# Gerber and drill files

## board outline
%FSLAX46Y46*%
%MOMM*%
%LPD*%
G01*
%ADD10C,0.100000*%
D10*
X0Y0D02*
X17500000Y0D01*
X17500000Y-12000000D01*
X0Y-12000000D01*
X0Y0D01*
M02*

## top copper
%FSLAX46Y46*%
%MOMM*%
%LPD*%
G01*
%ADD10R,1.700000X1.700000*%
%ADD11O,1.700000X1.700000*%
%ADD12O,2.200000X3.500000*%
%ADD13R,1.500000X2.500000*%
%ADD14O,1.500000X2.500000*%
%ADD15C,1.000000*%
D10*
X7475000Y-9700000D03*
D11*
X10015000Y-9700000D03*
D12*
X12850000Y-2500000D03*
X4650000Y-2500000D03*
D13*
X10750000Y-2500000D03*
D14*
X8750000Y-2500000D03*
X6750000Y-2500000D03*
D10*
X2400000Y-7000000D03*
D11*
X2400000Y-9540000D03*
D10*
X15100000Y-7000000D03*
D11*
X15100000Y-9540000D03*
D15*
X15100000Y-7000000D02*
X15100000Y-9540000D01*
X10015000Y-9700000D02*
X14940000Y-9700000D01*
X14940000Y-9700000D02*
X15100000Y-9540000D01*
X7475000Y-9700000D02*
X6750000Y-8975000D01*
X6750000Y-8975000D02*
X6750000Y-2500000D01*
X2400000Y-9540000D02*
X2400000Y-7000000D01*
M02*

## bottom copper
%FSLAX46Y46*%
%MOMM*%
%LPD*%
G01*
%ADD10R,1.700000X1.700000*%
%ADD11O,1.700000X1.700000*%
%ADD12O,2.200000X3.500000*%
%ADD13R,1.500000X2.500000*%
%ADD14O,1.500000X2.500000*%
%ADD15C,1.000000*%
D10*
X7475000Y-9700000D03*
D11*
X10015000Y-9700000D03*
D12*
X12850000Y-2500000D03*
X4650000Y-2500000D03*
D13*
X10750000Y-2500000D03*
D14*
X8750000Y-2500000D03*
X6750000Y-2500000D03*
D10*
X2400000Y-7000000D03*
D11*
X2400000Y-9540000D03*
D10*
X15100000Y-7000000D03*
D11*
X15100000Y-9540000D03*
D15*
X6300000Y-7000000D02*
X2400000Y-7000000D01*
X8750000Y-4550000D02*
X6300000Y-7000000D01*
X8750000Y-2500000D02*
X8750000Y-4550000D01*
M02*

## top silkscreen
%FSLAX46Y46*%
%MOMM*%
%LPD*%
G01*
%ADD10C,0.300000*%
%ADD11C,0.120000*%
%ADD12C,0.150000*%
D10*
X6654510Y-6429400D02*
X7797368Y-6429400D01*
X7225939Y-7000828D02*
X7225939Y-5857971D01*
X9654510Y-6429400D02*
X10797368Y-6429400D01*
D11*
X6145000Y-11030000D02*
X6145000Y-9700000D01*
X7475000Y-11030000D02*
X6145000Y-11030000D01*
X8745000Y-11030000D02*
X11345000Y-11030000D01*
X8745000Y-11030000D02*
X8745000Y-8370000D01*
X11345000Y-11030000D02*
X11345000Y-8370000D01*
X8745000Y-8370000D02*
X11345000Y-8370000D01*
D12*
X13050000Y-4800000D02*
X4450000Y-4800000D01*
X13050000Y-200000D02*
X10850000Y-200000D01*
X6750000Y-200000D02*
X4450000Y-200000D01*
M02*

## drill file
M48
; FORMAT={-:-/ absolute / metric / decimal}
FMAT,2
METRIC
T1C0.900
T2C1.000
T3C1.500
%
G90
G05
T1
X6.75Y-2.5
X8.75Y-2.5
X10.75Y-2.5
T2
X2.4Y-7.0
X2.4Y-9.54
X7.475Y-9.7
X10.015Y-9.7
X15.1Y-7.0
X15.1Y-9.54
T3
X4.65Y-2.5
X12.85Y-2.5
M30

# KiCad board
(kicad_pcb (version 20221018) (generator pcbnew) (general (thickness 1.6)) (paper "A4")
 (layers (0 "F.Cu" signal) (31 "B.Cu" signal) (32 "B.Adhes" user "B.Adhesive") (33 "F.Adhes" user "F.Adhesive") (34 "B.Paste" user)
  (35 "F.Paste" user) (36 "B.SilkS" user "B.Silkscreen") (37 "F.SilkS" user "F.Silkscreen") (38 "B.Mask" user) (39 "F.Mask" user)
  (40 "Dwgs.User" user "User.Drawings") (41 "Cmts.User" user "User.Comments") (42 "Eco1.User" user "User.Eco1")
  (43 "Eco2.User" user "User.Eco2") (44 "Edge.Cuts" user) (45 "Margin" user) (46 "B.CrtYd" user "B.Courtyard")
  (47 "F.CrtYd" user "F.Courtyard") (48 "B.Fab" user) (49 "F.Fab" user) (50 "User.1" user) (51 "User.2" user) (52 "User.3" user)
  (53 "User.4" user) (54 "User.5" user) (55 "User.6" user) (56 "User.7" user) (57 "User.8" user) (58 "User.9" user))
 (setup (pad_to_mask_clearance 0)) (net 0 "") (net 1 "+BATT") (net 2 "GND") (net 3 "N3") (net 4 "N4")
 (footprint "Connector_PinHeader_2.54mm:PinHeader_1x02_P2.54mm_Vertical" (layer "F.Cu") (at 7.475 9.7 90)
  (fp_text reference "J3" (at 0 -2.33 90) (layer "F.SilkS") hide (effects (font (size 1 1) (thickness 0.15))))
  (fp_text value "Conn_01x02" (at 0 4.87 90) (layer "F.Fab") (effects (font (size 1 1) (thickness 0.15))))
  (fp_line (start -1.33 -1.33) (end 0 -1.33) (stroke (width 0.12) (type solid)) (layer "F.SilkS"))
  (fp_line (start -1.33 0) (end -1.33 -1.33) (stroke (width 0.12) (type solid)) (layer "F.SilkS"))
  (fp_line (start -1.33 1.27) (end -1.33 3.87) (stroke (width 0.12) (type solid)) (layer "F.SilkS"))
  (fp_line (start -1.33 1.27) (end 1.33 1.27) (stroke (width 0.12) (type solid)) (layer "F.SilkS"))
  (fp_line (start -1.33 3.87) (end 1.33 3.87) (stroke (width 0.12) (type solid)) (layer "F.SilkS"))
  (fp_line (start 1.33 1.27) (end 1.33 3.87) (stroke (width 0.12) (type solid)) (layer "F.SilkS"))
  (pad "1" thru_hole rect (at 0 0 90) (size 1.7 1.7) (drill 1) (layers "*.Cu" "*.Mask") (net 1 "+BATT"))
  (pad "2" thru_hole oval (at 0 2.54 90) (size 1.7 1.7) (drill 1) (layers "*.Cu" "*.Mask") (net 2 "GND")))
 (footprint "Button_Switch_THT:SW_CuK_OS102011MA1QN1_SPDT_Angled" (layer "F.Cu") (at 10.75 2.5 180)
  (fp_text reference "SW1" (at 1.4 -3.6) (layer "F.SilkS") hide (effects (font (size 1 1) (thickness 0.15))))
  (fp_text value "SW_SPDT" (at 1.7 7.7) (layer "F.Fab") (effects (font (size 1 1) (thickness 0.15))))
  (fp_line (start -2.3 -2.3) (end 6.3 -2.3) (stroke (width 0.15) (type solid)) (layer "F.SilkS"))
  (fp_line (start -2.3 2.3) (end -0.1 2.3) (stroke (width 0.15) (type solid)) (layer "F.SilkS"))
  (fp_line (start 4 2.3) (end 6.3 2.3) (stroke (width 0.15) (type solid)) (layer "F.SilkS"))
  (pad "" thru_hole oval (at -2.1 0 180) (size 2.2 3.5) (drill 1.5) (layers "*.Cu" "*.Mask"))
  (pad "" thru_hole oval (at 6.1 0 180) (size 2.2 3.5) (drill 1.5) (layers "*.Cu" "*.Mask"))
  (pad "1" thru_hole rect (at 0 0 180) (size 1.5 2.5) (drill 0.9) (layers "*.Cu" "*.Mask") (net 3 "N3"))
  (pad "2" thru_hole oval (at 2 0 180) (size 1.5 2.5) (drill 0.9) (layers "*.Cu" "*.Mask") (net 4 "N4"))
  (pad "3" thru_hole oval (at 4 0 180) (size 1.5 2.5) (drill 0.9) (layers "*.Cu" "*.Mask") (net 1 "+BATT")))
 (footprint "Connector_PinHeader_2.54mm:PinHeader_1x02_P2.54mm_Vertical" (layer "B.Cu") (at 2.4 7 180)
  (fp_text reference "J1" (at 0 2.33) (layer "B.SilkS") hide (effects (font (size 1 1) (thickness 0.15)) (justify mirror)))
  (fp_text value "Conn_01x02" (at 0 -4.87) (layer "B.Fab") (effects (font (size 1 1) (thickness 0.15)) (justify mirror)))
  (pad "1" thru_hole rect (at 0 0 180) (size 1.7 1.7) (drill 1) (layers "*.Cu" "*.Mask") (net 4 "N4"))
  (pad "2" thru_hole oval (at 0 -2.54 180) (size 1.7 1.7) (drill 1) (layers "*.Cu" "*.Mask") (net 4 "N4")))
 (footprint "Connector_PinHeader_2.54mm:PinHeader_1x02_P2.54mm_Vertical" (layer "B.Cu") (at 15.1 7 180)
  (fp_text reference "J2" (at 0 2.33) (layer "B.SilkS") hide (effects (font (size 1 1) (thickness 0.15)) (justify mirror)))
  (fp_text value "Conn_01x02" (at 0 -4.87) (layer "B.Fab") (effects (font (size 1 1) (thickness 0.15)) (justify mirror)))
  (pad "1" thru_hole rect (at 0 0 180) (size 1.7 1.7) (drill 1) (layers "*.Cu" "*.Mask") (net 2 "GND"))
  (pad "2" thru_hole oval (at 0 -2.54 180) (size 1.7 1.7) (drill 1) (layers "*.Cu" "*.Mask") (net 2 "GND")))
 (gr_rect (start 0 0) (end 17.5 12) (stroke (width 0.1) (type default)) (fill none) (layer "Edge.Cuts"))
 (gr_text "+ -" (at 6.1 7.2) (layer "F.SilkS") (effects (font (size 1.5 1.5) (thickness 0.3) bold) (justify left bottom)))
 (segment (start 15.1 7) (end 15.1 9.54) (width 1) (layer "F.Cu") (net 2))
 (segment (start 10.015 9.7) (end 14.94 9.7) (width 1) (layer "F.Cu") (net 2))
 (segment (start 14.94 9.7) (end 15.1 9.54) (width 1) (layer "F.Cu") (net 2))
 (segment (start 7.475 9.7) (end 6.75 8.975) (width 1) (layer "F.Cu") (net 1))
 (segment (start 6.75 8.975) (end 6.75 2.5) (width 1) (layer "F.Cu") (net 1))
 (segment (start 2.4 9.54) (end 2.4 7) (width 1) (layer "F.Cu") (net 4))
 (segment (start 6.3 7) (end 2.4 7) (width 1) (layer "B.Cu") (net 4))
 (segment (start 8.75 4.55) (end 6.3 7) (width 1) (layer "B.Cu") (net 4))
 (segment (start 8.75 2.5) (end 8.75 4.55) (width 1) (layer "B.Cu") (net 4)))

